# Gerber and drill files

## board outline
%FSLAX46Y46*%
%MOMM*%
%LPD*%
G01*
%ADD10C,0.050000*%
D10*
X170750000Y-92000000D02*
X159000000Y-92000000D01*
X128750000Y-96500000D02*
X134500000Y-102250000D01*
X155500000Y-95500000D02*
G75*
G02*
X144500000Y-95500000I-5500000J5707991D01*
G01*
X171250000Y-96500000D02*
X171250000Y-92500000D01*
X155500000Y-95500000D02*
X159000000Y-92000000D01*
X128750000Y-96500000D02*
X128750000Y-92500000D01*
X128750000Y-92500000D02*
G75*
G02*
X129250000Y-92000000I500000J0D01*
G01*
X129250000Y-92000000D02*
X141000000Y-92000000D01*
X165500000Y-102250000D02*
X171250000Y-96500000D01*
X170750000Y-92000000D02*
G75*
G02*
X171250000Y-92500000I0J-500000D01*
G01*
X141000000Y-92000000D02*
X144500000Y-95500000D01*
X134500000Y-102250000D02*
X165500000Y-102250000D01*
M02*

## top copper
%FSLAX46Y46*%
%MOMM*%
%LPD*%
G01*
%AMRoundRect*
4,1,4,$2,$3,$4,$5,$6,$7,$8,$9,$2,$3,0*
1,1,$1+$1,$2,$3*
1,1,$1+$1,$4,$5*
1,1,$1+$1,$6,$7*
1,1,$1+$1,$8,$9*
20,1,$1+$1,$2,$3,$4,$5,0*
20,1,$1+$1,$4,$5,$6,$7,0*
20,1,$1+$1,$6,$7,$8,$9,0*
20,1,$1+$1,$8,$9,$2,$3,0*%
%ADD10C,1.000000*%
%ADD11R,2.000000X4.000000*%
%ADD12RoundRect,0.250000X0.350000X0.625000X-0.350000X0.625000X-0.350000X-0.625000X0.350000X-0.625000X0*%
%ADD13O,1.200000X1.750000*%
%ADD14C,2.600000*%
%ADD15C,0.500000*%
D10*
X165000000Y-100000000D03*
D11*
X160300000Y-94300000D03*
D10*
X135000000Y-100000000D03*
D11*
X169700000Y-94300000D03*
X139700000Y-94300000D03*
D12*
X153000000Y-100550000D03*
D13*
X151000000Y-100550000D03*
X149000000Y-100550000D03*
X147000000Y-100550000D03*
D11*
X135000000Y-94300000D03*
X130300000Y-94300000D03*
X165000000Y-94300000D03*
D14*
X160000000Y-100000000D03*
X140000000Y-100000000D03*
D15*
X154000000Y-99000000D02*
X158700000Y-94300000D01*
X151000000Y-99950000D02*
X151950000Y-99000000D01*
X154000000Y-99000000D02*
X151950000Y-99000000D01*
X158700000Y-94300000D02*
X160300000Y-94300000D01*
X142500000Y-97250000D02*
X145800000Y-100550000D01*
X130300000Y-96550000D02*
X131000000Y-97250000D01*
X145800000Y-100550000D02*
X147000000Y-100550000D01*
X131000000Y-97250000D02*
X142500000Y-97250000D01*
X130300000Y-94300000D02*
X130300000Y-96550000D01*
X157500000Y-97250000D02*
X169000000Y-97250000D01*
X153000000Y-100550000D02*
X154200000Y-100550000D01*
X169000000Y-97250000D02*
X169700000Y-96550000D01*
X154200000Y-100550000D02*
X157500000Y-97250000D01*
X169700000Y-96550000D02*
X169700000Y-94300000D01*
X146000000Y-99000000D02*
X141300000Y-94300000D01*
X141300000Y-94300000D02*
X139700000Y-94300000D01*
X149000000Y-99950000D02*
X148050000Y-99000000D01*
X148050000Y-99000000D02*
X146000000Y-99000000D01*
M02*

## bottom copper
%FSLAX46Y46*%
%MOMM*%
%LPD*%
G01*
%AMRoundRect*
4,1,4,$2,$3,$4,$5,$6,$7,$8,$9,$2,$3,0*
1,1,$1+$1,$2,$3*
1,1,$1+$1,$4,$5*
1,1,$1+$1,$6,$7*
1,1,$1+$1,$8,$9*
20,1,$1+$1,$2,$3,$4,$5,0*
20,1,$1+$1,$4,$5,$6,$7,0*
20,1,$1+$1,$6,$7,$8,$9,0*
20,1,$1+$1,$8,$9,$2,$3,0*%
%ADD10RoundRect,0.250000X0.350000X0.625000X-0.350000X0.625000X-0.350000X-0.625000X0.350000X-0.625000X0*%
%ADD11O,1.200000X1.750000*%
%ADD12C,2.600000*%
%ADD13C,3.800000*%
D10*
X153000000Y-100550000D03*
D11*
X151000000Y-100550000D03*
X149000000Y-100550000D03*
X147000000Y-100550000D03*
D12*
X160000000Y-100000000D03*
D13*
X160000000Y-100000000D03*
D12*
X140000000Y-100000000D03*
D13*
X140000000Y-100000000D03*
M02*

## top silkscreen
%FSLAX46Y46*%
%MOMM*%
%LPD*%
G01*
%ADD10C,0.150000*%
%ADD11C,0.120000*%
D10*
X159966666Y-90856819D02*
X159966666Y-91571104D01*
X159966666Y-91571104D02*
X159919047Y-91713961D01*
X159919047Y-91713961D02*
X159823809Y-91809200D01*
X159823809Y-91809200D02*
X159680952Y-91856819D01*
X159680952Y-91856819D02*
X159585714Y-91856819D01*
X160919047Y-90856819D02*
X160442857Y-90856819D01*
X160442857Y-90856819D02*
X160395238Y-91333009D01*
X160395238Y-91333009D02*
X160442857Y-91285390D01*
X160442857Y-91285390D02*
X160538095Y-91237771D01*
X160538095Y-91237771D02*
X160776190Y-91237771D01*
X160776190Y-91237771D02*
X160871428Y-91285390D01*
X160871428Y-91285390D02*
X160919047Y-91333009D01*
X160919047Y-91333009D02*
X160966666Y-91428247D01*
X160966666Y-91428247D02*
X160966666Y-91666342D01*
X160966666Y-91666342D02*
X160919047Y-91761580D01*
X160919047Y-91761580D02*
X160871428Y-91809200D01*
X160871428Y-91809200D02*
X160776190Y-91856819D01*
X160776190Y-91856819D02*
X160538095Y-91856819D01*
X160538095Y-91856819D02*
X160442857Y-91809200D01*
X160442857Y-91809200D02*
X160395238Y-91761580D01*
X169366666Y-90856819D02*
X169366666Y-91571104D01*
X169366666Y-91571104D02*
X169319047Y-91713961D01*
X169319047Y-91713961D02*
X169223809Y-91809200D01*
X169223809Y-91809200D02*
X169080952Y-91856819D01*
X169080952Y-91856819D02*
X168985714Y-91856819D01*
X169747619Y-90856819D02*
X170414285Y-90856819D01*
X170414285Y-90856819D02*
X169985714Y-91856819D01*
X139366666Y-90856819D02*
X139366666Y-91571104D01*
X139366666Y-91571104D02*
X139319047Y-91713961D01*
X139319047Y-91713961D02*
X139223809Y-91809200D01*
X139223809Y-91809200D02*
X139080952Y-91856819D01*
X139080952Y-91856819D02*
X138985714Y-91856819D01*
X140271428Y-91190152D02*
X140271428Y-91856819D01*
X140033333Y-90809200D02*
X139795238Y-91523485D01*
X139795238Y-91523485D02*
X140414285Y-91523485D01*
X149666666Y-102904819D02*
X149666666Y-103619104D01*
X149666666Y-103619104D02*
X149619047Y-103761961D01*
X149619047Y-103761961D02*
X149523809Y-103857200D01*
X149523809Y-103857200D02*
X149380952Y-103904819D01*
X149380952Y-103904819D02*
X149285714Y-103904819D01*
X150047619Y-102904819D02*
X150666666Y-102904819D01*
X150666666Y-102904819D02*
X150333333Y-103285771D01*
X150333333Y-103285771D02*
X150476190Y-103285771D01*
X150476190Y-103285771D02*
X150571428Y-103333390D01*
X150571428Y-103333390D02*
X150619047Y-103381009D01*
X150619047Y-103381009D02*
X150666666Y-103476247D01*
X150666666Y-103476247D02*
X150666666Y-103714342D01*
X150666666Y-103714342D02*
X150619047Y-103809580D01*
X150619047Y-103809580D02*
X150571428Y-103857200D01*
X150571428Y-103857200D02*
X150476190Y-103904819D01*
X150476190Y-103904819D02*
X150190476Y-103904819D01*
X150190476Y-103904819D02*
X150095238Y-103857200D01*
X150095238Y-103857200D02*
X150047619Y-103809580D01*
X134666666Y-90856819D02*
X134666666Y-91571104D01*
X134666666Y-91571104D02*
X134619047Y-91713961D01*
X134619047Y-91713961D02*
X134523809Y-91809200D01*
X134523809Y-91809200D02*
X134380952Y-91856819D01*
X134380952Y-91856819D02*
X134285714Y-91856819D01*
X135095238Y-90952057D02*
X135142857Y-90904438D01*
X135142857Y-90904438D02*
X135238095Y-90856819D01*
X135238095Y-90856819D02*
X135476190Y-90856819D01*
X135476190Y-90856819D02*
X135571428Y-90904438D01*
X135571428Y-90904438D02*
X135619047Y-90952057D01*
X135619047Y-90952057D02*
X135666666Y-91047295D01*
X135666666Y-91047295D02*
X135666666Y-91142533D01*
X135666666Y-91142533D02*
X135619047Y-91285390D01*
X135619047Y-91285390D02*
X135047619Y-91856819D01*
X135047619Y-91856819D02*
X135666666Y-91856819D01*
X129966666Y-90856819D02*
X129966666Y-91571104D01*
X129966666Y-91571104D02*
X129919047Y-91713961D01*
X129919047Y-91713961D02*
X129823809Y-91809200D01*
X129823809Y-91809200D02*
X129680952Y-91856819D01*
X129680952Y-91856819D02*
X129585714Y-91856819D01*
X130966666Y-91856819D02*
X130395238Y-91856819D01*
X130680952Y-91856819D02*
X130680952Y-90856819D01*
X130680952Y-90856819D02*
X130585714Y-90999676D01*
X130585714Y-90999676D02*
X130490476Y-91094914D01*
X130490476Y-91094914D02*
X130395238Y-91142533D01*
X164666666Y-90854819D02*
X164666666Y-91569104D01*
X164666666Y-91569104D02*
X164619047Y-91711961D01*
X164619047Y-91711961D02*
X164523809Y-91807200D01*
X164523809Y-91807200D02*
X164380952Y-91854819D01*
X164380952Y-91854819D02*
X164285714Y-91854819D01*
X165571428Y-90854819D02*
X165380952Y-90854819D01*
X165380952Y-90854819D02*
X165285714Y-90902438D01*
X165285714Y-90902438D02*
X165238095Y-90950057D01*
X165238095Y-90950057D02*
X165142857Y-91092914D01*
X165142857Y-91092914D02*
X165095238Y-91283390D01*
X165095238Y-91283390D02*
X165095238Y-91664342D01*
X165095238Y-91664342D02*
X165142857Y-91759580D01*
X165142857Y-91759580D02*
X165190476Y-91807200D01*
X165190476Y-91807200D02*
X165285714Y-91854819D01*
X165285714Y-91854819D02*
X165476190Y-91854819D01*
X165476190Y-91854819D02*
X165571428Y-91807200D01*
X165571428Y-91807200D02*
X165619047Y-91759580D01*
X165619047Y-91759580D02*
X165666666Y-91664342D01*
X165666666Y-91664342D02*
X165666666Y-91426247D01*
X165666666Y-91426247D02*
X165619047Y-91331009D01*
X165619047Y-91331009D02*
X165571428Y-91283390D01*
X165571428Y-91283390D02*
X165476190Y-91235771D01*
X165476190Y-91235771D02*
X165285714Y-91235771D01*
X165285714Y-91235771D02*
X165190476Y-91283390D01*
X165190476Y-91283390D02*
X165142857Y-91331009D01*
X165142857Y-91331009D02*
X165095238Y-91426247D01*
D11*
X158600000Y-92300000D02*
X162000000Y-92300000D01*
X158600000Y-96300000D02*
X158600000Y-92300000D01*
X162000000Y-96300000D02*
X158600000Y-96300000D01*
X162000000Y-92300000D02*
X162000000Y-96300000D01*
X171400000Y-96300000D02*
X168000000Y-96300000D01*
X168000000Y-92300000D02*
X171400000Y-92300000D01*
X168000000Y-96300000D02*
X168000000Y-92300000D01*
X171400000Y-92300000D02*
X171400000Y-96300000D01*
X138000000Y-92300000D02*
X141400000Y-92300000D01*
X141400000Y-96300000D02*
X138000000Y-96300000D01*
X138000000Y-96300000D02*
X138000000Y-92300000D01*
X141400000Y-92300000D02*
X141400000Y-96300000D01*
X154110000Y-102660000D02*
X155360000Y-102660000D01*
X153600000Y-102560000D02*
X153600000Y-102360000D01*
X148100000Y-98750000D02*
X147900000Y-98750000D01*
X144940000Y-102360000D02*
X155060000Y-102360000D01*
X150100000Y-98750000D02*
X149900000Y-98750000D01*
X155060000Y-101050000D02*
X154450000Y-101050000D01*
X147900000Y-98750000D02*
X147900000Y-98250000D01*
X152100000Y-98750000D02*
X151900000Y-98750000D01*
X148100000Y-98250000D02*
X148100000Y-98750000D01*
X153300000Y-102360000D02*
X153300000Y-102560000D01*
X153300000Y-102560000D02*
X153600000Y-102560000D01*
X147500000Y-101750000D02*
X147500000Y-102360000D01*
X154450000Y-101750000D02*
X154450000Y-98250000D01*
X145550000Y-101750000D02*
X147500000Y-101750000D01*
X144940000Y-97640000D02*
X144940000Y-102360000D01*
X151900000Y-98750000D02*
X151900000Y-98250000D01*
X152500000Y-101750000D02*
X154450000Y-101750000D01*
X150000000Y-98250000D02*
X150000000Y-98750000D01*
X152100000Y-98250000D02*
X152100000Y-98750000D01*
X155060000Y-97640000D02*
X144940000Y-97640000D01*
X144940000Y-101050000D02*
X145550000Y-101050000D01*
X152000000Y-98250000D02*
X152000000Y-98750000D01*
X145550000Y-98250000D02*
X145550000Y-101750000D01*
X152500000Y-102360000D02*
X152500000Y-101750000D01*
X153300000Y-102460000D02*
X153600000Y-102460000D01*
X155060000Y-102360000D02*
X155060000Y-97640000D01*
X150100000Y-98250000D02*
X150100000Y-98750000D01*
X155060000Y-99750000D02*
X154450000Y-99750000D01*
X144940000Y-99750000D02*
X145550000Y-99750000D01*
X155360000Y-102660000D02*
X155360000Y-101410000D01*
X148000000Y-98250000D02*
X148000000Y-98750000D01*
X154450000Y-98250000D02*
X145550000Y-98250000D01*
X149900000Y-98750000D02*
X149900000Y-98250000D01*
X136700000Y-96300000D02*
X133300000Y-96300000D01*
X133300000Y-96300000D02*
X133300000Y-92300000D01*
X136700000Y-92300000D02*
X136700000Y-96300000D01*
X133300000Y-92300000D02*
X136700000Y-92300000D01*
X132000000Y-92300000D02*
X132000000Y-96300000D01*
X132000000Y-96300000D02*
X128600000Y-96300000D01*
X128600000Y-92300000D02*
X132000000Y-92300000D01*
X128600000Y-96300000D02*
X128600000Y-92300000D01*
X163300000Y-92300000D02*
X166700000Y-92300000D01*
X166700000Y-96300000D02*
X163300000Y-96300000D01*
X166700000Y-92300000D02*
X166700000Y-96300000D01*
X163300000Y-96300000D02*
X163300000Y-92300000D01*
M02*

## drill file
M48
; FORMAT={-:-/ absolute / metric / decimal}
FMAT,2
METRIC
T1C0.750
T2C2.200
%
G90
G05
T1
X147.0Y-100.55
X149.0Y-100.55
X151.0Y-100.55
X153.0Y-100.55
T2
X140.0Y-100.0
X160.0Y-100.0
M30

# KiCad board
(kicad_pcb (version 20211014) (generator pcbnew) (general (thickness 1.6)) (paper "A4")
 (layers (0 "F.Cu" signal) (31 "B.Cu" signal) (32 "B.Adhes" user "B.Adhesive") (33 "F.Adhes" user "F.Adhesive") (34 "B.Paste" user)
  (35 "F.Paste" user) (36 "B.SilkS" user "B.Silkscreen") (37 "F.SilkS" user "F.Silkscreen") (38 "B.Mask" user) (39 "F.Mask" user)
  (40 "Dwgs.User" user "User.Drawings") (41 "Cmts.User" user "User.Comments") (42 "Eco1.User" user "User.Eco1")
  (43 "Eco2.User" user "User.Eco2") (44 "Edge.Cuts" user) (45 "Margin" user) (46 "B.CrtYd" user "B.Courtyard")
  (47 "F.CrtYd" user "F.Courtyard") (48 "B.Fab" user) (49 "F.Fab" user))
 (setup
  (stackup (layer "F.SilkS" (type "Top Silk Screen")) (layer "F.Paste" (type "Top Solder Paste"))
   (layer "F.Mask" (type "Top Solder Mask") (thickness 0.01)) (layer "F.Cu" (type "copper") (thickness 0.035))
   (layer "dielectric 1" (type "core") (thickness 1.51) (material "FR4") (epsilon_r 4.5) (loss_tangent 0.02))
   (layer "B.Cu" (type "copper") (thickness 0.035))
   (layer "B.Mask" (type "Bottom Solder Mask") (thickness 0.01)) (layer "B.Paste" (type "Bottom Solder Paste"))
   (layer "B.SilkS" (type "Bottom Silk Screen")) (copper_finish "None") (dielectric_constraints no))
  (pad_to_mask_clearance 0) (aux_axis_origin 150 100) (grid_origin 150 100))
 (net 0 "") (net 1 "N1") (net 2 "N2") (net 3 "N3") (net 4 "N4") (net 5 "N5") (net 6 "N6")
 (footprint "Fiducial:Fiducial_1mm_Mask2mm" (layer "F.Cu") (at 165 100)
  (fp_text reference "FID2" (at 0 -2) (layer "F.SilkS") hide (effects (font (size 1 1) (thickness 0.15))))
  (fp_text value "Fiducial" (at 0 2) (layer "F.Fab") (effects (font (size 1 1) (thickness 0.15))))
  (pad "" smd circle (at 0 0) (size 1 1) (layers "F.Cu" "F.Mask") (solder_mask_margin 0.5) (clearance 0.5)))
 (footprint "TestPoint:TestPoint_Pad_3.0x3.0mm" (layer "F.Cu") (at 160.3 93.8)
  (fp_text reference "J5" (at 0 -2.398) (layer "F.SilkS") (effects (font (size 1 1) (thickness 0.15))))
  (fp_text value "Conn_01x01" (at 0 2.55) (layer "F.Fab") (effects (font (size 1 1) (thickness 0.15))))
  (fp_line (start -1.7 -1.5) (end 1.7 -1.5) (layer "F.SilkS") (width 0.12))
  (fp_line (start -1.7 2.5) (end -1.7 -1.5) (layer "F.SilkS") (width 0.12))
  (fp_line (start 1.7 2.5) (end -1.7 2.5) (layer "F.SilkS") (width 0.12))
  (fp_line (start 1.7 -1.5) (end 1.7 2.5) (layer "F.SilkS") (width 0.12))
  (pad "1" smd rect (at 0 0.5) (size 2 4) (layers "F.Cu" "F.Mask") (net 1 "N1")))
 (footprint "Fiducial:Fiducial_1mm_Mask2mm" (layer "F.Cu") (at 135 100)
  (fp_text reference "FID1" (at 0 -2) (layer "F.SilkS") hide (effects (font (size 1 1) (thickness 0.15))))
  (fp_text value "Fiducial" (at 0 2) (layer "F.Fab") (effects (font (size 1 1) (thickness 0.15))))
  (pad "" smd circle (at 0 0) (size 1 1) (layers "F.Cu" "F.Mask") (solder_mask_margin 0.5) (clearance 0.5)))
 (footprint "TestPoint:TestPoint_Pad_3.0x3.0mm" (layer "F.Cu") (at 169.7 93.8)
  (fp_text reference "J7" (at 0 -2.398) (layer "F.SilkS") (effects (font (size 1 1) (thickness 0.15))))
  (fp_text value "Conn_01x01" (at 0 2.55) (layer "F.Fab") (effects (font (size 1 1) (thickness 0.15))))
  (fp_line (start 1.7 2.5) (end -1.7 2.5) (layer "F.SilkS") (width 0.12))
  (fp_line (start -1.7 -1.5) (end 1.7 -1.5) (layer "F.SilkS") (width 0.12))
  (fp_line (start -1.7 2.5) (end -1.7 -1.5) (layer "F.SilkS") (width 0.12))
  (fp_line (start 1.7 -1.5) (end 1.7 2.5) (layer "F.SilkS") (width 0.12))
  (pad "1" smd rect (at 0 0.5) (size 2 4) (layers "F.Cu" "F.Mask") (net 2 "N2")))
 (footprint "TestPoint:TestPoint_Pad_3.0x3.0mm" (layer "F.Cu") (at 139.7 93.8)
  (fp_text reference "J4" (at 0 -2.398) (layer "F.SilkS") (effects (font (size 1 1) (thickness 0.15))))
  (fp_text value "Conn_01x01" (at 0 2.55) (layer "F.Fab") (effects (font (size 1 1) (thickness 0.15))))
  (fp_line (start -1.7 -1.5) (end 1.7 -1.5) (layer "F.SilkS") (width 0.12))
  (fp_line (start 1.7 2.5) (end -1.7 2.5) (layer "F.SilkS") (width 0.12))
  (fp_line (start -1.7 2.5) (end -1.7 -1.5) (layer "F.SilkS") (width 0.12))
  (fp_line (start 1.7 -1.5) (end 1.7 2.5) (layer "F.SilkS") (width 0.12))
  (pad "1" smd rect (at 0 0.5) (size 2 4) (layers "F.Cu" "F.Mask") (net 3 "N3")))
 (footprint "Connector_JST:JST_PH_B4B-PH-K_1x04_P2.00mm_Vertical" (layer "F.Cu") (at 153 100.55 180)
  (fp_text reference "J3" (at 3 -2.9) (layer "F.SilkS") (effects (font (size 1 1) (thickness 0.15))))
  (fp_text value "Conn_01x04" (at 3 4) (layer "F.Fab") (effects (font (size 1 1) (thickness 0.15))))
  (fp_line (start -1.11 -2.11) (end -2.36 -2.11) (layer "F.SilkS") (width 0.12))
  (fp_line (start -0.6 -2.01) (end -0.6 -1.81) (layer "F.SilkS") (width 0.12))
  (fp_line (start 4.9 1.8) (end 5.1 1.8) (layer "F.SilkS") (width 0.12))
  (fp_line (start 8.06 -1.81) (end -2.06 -1.81) (layer "F.SilkS") (width 0.12))
  (fp_line (start 2.9 1.8) (end 3.1 1.8) (layer "F.SilkS") (width 0.12))
  (fp_line (start -2.06 -0.5) (end -1.45 -0.5) (layer "F.SilkS") (width 0.12))
  (fp_line (start 5.1 1.8) (end 5.1 2.3) (layer "F.SilkS") (width 0.12))
  (fp_line (start 0.9 1.8) (end 1.1 1.8) (layer "F.SilkS") (width 0.12))
  (fp_line (start 4.9 2.3) (end 4.9 1.8) (layer "F.SilkS") (width 0.12))
  (fp_line (start -0.3 -1.81) (end -0.3 -2.01) (layer "F.SilkS") (width 0.12))
  (fp_line (start -0.3 -2.01) (end -0.6 -2.01) (layer "F.SilkS") (width 0.12))
  (fp_line (start 5.5 -1.2) (end 5.5 -1.81) (layer "F.SilkS") (width 0.12))
  (fp_line (start -1.45 -1.2) (end -1.45 2.3) (layer "F.SilkS") (width 0.12))
  (fp_line (start 7.45 -1.2) (end 5.5 -1.2) (layer "F.SilkS") (width 0.12))
  (fp_line (start 8.06 2.91) (end 8.06 -1.81) (layer "F.SilkS") (width 0.12))
  (fp_line (start 1.1 1.8) (end 1.1 2.3) (layer "F.SilkS") (width 0.12))
  (fp_line (start 0.5 -1.2) (end -1.45 -1.2) (layer "F.SilkS") (width 0.12))
  (fp_line (start 3 2.3) (end 3 1.8) (layer "F.SilkS") (width 0.12))
  (fp_line (start 0.9 2.3) (end 0.9 1.8) (layer "F.SilkS") (width 0.12))
  (fp_line (start -2.06 2.91) (end 8.06 2.91) (layer "F.SilkS") (width 0.12))
  (fp_line (start 8.06 -0.5) (end 7.45 -0.5) (layer "F.SilkS") (width 0.12))
  (fp_line (start 1 2.3) (end 1 1.8) (layer "F.SilkS") (width 0.12))
  (fp_line (start 7.45 2.3) (end 7.45 -1.2) (layer "F.SilkS") (width 0.12))
  (fp_line (start 0.5 -1.81) (end 0.5 -1.2) (layer "F.SilkS") (width 0.12))
  (fp_line (start -0.3 -1.91) (end -0.6 -1.91) (layer "F.SilkS") (width 0.12))
  (fp_line (start -2.06 -1.81) (end -2.06 2.91) (layer "F.SilkS") (width 0.12))
  (fp_line (start 2.9 2.3) (end 2.9 1.8) (layer "F.SilkS") (width 0.12))
  (fp_line (start -2.06 0.8) (end -1.45 0.8) (layer "F.SilkS") (width 0.12))
  (fp_line (start 8.06 0.8) (end 7.45 0.8) (layer "F.SilkS") (width 0.12))
  (fp_line (start -2.36 -2.11) (end -2.36 -0.86) (layer "F.SilkS") (width 0.12))
  (fp_line (start 5 2.3) (end 5 1.8) (layer "F.SilkS") (width 0.12))
  (fp_line (start -1.45 2.3) (end 7.45 2.3) (layer "F.SilkS") (width 0.12))
  (fp_line (start 3.1 1.8) (end 3.1 2.3) (layer "F.SilkS") (width 0.12))
  (pad "1" thru_hole roundrect (at 0 0 180) (size 1.2 1.75) (drill 0.75) (layers *.Cu *.Mask) (roundrect_rratio 0.2083333333) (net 2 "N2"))
  (pad "2" thru_hole oval (at 2 0 180) (size 1.2 1.75) (drill 0.75) (layers *.Cu *.Mask) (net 1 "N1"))
  (pad "3" thru_hole oval (at 4 0 180) (size 1.2 1.75) (drill 0.75) (layers *.Cu *.Mask) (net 3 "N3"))
  (pad "4" thru_hole oval (at 6 0 180) (size 1.2 1.75) (drill 0.75) (layers *.Cu *.Mask) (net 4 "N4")))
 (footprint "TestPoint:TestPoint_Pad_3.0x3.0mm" (layer "F.Cu") (at 135 93.8)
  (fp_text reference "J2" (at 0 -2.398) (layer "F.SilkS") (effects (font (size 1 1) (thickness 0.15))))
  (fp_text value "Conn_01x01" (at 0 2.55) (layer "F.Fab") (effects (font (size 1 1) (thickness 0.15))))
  (fp_line (start 1.7 2.5) (end -1.7 2.5) (layer "F.SilkS") (width 0.12))
  (fp_line (start -1.7 2.5) (end -1.7 -1.5) (layer "F.SilkS") (width 0.12))
  (fp_line (start 1.7 -1.5) (end 1.7 2.5) (layer "F.SilkS") (width 0.12))
  (fp_line (start -1.7 -1.5) (end 1.7 -1.5) (layer "F.SilkS") (width 0.12))
  (pad "1" smd rect (at 0 0.5) (size 2 4) (layers "F.Cu" "F.Mask") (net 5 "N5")))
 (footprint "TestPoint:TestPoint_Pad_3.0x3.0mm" (layer "F.Cu") (at 130.3 93.8)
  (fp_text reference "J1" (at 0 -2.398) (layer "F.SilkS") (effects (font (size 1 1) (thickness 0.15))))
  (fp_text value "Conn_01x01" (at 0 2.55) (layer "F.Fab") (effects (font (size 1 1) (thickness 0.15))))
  (fp_line (start 1.7 -1.5) (end 1.7 2.5) (layer "F.SilkS") (width 0.12))
  (fp_line (start 1.7 2.5) (end -1.7 2.5) (layer "F.SilkS") (width 0.12))
  (fp_line (start -1.7 -1.5) (end 1.7 -1.5) (layer "F.SilkS") (width 0.12))
  (fp_line (start -1.7 2.5) (end -1.7 -1.5) (layer "F.SilkS") (width 0.12))
  (pad "1" smd rect (at 0 0.5) (size 2 4) (layers "F.Cu" "F.Mask") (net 4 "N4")))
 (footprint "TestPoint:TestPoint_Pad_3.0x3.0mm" (layer "F.Cu") (at 165 94.3)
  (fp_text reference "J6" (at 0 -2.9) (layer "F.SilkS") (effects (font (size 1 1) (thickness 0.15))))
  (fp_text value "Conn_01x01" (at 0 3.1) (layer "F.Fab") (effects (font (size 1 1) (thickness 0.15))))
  (fp_line (start -1.7 -2) (end 1.7 -2) (layer "F.SilkS") (width 0.12))
  (fp_line (start 1.7 2) (end -1.7 2) (layer "F.SilkS") (width 0.12))
  (fp_line (start 1.7 -2) (end 1.7 2) (layer "F.SilkS") (width 0.12))
  (fp_line (start -1.7 2) (end -1.7 -2) (layer "F.SilkS") (width 0.12))
  (pad "1" smd rect (at 0 0) (size 2 4) (layers "F.Cu" "F.Mask") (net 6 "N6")))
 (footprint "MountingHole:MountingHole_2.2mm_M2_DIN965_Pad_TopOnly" (layer "B.Cu") (at 160 100 180)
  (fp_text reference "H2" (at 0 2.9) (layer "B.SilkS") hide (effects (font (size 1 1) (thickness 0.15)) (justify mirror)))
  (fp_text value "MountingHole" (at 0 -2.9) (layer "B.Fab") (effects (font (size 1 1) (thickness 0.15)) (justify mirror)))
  (pad "1" thru_hole circle (at 0 0 180) (size 2.6 2.6) (drill 2.2) (layers *.Cu *.Mask))
  (pad "1" connect circle (at 0 0 180) (size 3.8 3.8) (layers "B.Cu" "B.Mask")))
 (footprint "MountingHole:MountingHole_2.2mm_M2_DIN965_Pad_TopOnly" (layer "B.Cu") (at 140 100 180)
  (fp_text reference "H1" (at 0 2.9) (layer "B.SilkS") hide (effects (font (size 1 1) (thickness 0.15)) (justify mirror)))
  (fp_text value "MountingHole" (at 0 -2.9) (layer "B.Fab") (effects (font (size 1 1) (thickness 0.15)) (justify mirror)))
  (pad "1" thru_hole circle (at 0 0 180) (size 2.6 2.6) (drill 2.2) (layers *.Cu *.Mask))
  (pad "1" connect circle (at 0 0 180) (size 3.8 3.8) (layers "B.Cu" "B.Mask")))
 (gr_line (start 170.75 92) (end 159 92) (layer "Edge.Cuts") (width 0.05))
 (gr_line (start 128.75 96.5) (end 134.5 102.25) (layer "Edge.Cuts") (width 0.05))
 (gr_arc (start 155.5 95.5) (mid 150 97.71862) (end 144.5 95.5) (layer "Edge.Cuts") (width 0.05))
 (gr_line (start 171.25 96.5) (end 171.25 92.5) (layer "Edge.Cuts") (width 0.05))
 (gr_line (start 155.5 95.5) (end 159 92) (layer "Edge.Cuts") (width 0.05))
 (gr_line (start 128.75 96.5) (end 128.75 92.5) (layer "Edge.Cuts") (width 0.05))
 (gr_arc (start 128.75 92.5) (mid 128.896447 92.146447) (end 129.25 92) (layer "Edge.Cuts") (width 0.05))
 (gr_line (start 129.25 92) (end 141 92) (layer "Edge.Cuts") (width 0.05))
 (gr_line (start 165.5 102.25) (end 171.25 96.5) (layer "Edge.Cuts") (width 0.05))
 (gr_arc (start 170.75 92) (mid 171.103553 92.146447) (end 171.25 92.5) (layer "Edge.Cuts") (width 0.05))
 (gr_line (start 141 92) (end 144.5 95.5) (layer "Edge.Cuts") (width 0.05))
 (gr_line (start 134.5 102.25) (end 165.5 102.25) (layer "Edge.Cuts") (width 0.05))
 (segment (start 154 99) (end 158.7 94.3) (width 0.5) (layer "F.Cu") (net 1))
 (segment (start 151 99.95) (end 151.95 99) (width 0.5) (layer "F.Cu") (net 1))
 (segment (start 154 99) (end 151.95 99) (width 0.5) (layer "F.Cu") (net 1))
 (segment (start 158.7 94.3) (end 160.3 94.3) (width 0.5) (layer "F.Cu") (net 1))
 (segment (start 142.5 97.25) (end 145.8 100.55) (width 0.5) (layer "F.Cu") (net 4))
 (segment (start 130.3 96.55) (end 131 97.25) (width 0.5) (layer "F.Cu") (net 4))
 (segment (start 145.8 100.55) (end 147 100.55) (width 0.5) (layer "F.Cu") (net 4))
 (segment (start 131 97.25) (end 142.5 97.25) (width 0.5) (layer "F.Cu") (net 4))
 (segment (start 130.3 94.3) (end 130.3 96.55) (width 0.5) (layer "F.Cu") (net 4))
 (segment (start 157.5 97.25) (end 169 97.25) (width 0.5) (layer "F.Cu") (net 2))
 (segment (start 153 100.55) (end 154.2 100.55) (width 0.5) (layer "F.Cu") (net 2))
 (segment (start 169 97.25) (end 169.7 96.55) (width 0.5) (layer "F.Cu") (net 2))
 (segment (start 154.2 100.55) (end 157.5 97.25) (width 0.5) (layer "F.Cu") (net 2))
 (segment (start 169.7 96.55) (end 169.7 94.3) (width 0.5) (layer "F.Cu") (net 2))
 (segment (start 146 99) (end 141.3 94.3) (width 0.5) (layer "F.Cu") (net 3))
 (segment (start 141.3 94.3) (end 139.7 94.3) (width 0.5) (layer "F.Cu") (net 3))
 (segment (start 149 99.95) (end 148.05 99) (width 0.5) (layer "F.Cu") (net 3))
 (segment (start 148.05 99) (end 146 99) (width 0.5) (layer "F.Cu") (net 3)))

